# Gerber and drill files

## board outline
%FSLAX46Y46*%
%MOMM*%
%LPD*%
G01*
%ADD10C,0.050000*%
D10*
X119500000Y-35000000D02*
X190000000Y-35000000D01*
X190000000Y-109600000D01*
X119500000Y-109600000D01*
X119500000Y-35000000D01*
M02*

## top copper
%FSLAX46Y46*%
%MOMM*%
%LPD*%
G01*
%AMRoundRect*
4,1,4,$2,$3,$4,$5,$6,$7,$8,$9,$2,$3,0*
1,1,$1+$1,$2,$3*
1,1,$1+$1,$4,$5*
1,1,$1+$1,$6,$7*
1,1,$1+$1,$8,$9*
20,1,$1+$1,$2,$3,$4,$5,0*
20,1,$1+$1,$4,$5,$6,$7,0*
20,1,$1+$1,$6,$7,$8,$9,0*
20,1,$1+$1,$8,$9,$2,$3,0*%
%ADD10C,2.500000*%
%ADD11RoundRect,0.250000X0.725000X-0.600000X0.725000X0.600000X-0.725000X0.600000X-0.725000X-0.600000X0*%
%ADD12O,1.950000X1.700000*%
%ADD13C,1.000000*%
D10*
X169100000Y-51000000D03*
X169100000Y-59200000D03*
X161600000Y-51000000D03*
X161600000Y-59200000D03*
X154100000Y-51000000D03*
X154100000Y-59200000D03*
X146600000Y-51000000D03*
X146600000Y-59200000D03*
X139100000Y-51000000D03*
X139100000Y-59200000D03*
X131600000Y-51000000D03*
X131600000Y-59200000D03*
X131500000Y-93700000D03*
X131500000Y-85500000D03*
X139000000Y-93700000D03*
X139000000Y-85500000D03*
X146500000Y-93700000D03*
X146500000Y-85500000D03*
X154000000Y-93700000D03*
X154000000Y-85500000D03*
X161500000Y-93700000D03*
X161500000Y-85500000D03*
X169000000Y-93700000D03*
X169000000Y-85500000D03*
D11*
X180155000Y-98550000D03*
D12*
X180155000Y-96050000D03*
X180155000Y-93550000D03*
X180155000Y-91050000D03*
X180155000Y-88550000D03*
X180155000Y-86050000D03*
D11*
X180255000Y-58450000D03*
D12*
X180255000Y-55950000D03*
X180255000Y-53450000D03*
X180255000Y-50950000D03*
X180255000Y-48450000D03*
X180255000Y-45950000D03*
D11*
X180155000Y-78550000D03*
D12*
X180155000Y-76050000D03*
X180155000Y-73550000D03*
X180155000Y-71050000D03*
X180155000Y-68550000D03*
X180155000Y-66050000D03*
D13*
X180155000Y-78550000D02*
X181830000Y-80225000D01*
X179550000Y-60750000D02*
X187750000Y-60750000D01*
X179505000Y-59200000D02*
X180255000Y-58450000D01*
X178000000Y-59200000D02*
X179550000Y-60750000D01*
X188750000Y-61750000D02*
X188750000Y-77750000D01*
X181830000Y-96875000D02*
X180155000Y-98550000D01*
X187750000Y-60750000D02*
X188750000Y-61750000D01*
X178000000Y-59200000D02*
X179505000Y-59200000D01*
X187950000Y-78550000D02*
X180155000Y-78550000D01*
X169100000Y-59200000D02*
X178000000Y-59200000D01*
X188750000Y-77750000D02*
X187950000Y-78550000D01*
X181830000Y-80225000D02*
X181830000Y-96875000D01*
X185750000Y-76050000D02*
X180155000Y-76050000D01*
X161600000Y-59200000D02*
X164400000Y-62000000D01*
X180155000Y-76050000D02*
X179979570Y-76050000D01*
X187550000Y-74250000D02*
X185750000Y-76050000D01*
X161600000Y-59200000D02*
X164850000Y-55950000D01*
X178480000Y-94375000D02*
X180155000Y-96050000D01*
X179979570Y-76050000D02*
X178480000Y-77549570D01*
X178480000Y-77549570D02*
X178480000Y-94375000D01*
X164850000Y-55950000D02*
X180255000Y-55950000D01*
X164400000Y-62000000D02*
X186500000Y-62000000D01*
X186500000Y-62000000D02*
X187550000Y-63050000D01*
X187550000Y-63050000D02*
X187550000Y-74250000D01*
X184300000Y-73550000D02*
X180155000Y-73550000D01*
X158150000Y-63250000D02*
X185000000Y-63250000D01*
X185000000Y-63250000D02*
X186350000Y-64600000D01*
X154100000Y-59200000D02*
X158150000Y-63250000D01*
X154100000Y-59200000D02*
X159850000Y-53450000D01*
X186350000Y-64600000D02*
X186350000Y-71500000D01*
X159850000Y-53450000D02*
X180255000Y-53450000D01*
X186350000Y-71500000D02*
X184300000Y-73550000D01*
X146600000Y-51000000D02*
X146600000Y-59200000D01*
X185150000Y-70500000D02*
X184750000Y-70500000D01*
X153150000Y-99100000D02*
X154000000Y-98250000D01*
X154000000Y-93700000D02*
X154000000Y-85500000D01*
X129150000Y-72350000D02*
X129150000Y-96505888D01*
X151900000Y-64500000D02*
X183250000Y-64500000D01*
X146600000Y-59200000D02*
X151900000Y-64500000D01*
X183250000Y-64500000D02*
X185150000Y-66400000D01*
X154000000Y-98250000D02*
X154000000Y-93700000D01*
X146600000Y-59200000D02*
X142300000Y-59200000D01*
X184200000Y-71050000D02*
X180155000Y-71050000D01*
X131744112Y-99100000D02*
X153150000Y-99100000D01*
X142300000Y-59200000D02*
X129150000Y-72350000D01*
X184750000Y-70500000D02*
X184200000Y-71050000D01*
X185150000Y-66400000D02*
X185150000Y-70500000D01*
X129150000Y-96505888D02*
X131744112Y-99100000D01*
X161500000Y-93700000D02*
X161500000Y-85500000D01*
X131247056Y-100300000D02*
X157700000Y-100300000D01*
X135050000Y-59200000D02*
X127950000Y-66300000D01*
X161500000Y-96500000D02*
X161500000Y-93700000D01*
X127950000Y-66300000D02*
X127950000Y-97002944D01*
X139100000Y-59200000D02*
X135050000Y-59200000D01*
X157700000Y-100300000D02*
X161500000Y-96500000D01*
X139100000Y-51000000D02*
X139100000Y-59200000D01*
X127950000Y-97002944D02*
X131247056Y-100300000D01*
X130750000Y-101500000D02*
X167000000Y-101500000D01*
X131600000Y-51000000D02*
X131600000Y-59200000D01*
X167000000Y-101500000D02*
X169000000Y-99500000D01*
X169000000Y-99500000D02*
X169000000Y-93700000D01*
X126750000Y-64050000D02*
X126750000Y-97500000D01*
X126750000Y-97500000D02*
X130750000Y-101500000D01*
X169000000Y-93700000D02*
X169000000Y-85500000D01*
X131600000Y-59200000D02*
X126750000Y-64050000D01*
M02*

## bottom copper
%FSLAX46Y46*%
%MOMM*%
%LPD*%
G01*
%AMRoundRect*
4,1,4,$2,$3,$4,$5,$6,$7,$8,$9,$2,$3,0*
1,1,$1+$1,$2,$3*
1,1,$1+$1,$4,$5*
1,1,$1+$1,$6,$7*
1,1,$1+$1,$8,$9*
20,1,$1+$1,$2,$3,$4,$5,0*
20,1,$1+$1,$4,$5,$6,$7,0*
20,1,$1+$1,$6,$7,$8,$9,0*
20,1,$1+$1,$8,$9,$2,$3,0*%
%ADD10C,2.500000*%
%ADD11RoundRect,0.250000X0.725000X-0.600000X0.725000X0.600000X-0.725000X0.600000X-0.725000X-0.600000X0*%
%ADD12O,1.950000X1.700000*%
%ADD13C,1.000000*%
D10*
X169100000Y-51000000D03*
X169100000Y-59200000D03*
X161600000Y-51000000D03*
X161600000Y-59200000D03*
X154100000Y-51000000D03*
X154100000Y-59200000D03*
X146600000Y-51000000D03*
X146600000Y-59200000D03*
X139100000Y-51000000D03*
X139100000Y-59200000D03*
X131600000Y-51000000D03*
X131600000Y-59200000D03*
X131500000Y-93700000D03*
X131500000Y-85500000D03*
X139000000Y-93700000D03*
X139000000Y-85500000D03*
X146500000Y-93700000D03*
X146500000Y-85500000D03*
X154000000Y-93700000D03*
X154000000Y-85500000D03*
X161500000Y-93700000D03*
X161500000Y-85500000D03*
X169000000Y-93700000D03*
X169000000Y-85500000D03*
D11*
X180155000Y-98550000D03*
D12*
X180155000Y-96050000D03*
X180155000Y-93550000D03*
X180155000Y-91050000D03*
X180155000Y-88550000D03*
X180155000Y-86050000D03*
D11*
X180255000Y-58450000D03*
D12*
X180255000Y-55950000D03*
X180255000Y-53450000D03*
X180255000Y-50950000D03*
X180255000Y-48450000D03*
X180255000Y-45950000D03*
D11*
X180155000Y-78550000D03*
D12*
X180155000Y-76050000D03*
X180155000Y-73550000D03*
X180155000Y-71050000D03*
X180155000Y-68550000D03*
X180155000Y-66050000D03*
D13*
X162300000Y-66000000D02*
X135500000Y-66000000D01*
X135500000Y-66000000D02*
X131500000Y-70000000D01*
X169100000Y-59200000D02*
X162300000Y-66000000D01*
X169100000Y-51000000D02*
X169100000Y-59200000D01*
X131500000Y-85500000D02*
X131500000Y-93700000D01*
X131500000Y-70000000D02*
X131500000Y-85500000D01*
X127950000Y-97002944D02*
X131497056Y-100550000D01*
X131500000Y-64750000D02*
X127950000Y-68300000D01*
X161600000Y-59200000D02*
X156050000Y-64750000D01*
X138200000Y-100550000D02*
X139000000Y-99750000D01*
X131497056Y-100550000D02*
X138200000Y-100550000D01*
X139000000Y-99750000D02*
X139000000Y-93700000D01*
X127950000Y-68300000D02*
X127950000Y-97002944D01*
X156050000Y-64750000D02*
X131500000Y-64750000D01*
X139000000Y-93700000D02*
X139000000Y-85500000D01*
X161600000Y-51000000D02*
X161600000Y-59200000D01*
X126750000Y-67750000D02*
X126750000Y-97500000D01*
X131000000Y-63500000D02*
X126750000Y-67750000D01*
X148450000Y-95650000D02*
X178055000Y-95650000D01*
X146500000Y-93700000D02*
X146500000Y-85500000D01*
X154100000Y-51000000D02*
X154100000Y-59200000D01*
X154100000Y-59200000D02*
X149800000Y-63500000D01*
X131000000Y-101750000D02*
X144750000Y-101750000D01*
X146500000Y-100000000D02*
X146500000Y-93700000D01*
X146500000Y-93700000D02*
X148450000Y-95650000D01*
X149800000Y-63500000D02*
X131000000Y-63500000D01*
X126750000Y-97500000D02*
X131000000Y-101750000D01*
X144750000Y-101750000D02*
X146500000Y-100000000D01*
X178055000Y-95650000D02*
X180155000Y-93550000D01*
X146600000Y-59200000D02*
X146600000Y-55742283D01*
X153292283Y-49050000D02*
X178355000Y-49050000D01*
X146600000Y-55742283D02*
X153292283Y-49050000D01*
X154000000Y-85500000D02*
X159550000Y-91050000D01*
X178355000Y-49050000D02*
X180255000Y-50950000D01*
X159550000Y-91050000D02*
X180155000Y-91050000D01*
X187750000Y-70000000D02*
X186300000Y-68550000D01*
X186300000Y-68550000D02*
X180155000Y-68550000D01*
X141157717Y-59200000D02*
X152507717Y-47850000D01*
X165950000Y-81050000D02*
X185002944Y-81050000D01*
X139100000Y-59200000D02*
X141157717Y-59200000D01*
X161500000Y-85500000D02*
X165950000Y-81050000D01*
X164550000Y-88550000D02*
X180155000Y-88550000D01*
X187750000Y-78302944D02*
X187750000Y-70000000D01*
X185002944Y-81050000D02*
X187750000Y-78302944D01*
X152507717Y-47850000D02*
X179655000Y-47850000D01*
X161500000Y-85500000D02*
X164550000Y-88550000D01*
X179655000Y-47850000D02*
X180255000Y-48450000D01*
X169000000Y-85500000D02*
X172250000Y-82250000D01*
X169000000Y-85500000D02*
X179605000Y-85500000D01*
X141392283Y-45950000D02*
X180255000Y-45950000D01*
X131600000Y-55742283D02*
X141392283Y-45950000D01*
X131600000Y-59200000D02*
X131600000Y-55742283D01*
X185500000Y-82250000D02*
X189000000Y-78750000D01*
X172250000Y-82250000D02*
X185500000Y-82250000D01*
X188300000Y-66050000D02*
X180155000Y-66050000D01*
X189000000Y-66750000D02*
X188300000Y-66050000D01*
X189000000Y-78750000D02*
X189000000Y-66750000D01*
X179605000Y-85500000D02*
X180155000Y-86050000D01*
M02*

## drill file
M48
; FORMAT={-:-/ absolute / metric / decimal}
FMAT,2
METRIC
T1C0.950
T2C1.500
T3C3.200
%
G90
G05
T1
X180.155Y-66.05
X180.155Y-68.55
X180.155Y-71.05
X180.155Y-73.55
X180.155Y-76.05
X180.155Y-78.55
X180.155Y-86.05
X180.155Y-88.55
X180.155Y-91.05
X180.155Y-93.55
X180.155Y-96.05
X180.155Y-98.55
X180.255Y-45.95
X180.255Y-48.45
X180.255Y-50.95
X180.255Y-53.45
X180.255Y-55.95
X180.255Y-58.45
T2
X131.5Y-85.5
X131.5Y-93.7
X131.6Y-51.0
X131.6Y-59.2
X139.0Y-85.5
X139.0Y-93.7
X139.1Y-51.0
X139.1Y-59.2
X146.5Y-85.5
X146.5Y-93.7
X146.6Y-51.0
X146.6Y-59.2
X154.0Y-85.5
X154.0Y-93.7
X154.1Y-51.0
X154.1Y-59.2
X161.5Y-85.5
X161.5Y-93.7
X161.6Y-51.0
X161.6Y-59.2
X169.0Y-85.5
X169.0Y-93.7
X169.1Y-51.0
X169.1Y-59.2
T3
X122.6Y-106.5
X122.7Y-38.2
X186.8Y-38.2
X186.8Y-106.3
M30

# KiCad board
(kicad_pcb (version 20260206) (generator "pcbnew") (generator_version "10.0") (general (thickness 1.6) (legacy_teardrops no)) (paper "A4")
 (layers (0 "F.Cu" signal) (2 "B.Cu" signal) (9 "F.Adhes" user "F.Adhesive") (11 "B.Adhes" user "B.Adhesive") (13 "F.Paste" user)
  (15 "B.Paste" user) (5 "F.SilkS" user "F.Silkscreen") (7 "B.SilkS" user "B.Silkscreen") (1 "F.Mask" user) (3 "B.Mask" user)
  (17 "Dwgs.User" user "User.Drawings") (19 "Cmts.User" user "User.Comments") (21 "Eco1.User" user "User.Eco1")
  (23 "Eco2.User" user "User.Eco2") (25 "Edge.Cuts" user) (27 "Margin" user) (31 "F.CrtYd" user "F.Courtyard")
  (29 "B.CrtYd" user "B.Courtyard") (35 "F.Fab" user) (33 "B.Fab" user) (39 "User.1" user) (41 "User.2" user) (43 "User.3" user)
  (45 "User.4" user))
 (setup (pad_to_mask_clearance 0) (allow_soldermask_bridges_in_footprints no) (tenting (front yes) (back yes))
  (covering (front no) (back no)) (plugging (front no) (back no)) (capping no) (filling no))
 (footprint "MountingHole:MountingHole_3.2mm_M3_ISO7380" (layer "F.Cu") (at 122.6 106.5)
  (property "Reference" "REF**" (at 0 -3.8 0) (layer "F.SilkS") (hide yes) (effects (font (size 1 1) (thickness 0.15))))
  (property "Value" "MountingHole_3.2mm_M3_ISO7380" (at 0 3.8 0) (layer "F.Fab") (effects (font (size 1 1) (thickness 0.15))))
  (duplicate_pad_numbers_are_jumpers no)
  (pad "" np_thru_hole circle (at 0 0) (size 3.2 3.2) (drill 3.2) (layers "*.Cu" "*.Mask")))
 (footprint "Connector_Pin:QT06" (layer "F.Cu") (at 150.36 51.82)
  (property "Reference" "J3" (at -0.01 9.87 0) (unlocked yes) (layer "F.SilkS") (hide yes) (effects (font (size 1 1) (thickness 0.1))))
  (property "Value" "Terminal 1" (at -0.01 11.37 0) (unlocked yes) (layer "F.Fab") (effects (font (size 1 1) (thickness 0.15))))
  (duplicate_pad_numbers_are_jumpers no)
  (pad "1" thru_hole circle (at 18.74 -0.82) (size 2.5 2.5) (drill 1.5) (layers "*.Cu" "*.Mask") (remove_unused_layers no)
   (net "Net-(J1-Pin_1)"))
  (pad "1" thru_hole circle (at 18.74 7.38) (size 2.5 2.5) (drill 1.5) (layers "*.Cu" "*.Mask") (remove_unused_layers no)
   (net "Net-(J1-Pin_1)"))
  (pad "2" thru_hole circle (at 11.24 -0.82) (size 2.5 2.5) (drill 1.5) (layers "*.Cu" "*.Mask") (remove_unused_layers no)
   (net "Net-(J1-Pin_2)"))
  (pad "2" thru_hole circle (at 11.24 7.38) (size 2.5 2.5) (drill 1.5) (layers "*.Cu" "*.Mask") (remove_unused_layers no)
   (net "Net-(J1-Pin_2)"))
  (pad "3" thru_hole circle (at 3.74 -0.82) (size 2.5 2.5) (drill 1.5) (layers "*.Cu" "*.Mask") (remove_unused_layers no)
   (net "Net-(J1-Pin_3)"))
  (pad "3" thru_hole circle (at 3.74 7.38) (size 2.5 2.5) (drill 1.5) (layers "*.Cu" "*.Mask") (remove_unused_layers no)
   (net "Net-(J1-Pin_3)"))
  (pad "4" thru_hole circle (at -3.76 -0.82) (size 2.5 2.5) (drill 1.5) (layers "*.Cu" "*.Mask") (remove_unused_layers no)
   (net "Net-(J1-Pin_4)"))
  (pad "4" thru_hole circle (at -3.76 7.38) (size 2.5 2.5) (drill 1.5) (layers "*.Cu" "*.Mask") (remove_unused_layers no)
   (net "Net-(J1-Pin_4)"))
  (pad "5" thru_hole circle (at -11.26 -0.82) (size 2.5 2.5) (drill 1.5) (layers "*.Cu" "*.Mask") (remove_unused_layers no)
   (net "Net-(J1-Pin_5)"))
  (pad "5" thru_hole circle (at -11.26 7.38) (size 2.5 2.5) (drill 1.5) (layers "*.Cu" "*.Mask") (remove_unused_layers no)
   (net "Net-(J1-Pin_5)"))
  (pad "6" thru_hole circle (at -18.76 -0.82) (size 2.5 2.5) (drill 1.5) (layers "*.Cu" "*.Mask") (remove_unused_layers no)
   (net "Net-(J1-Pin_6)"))
  (pad "6" thru_hole circle (at -18.76 7.38) (size 2.5 2.5) (drill 1.5) (layers "*.Cu" "*.Mask") (remove_unused_layers no)
   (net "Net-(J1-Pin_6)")))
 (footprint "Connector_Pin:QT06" (layer "F.Cu") (at 150.24 92.88 180)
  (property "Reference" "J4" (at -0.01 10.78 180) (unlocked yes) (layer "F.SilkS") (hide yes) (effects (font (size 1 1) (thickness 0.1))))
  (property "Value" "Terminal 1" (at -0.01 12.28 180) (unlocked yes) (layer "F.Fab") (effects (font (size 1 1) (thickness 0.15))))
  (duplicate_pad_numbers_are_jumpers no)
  (pad "1" thru_hole circle (at 18.74 -0.82 180) (size 2.5 2.5) (drill 1.5) (layers "*.Cu" "*.Mask") (remove_unused_layers no)
   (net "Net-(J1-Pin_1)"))
  (pad "1" thru_hole circle (at 18.74 7.38 180) (size 2.5 2.5) (drill 1.5) (layers "*.Cu" "*.Mask") (remove_unused_layers no)
   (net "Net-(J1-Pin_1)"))
  (pad "2" thru_hole circle (at 11.24 -0.82 180) (size 2.5 2.5) (drill 1.5) (layers "*.Cu" "*.Mask") (remove_unused_layers no)
   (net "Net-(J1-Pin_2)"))
  (pad "2" thru_hole circle (at 11.24 7.38 180) (size 2.5 2.5) (drill 1.5) (layers "*.Cu" "*.Mask") (remove_unused_layers no)
   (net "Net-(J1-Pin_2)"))
  (pad "3" thru_hole circle (at 3.74 -0.82 180) (size 2.5 2.5) (drill 1.5) (layers "*.Cu" "*.Mask") (remove_unused_layers no)
   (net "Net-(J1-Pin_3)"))
  (pad "3" thru_hole circle (at 3.74 7.38 180) (size 2.5 2.5) (drill 1.5) (layers "*.Cu" "*.Mask") (remove_unused_layers no)
   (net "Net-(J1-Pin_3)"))
  (pad "4" thru_hole circle (at -3.76 -0.82 180) (size 2.5 2.5) (drill 1.5) (layers "*.Cu" "*.Mask") (remove_unused_layers no)
   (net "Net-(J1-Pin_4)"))
  (pad "4" thru_hole circle (at -3.76 7.38 180) (size 2.5 2.5) (drill 1.5) (layers "*.Cu" "*.Mask") (remove_unused_layers no)
   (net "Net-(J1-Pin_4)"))
  (pad "5" thru_hole circle (at -11.26 -0.82 180) (size 2.5 2.5) (drill 1.5) (layers "*.Cu" "*.Mask") (remove_unused_layers no)
   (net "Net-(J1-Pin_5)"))
  (pad "5" thru_hole circle (at -11.26 7.38 180) (size 2.5 2.5) (drill 1.5) (layers "*.Cu" "*.Mask") (remove_unused_layers no)
   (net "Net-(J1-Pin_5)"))
  (pad "6" thru_hole circle (at -18.76 -0.82 180) (size 2.5 2.5) (drill 1.5) (layers "*.Cu" "*.Mask") (remove_unused_layers no)
   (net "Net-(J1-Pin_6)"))
  (pad "6" thru_hole circle (at -18.76 7.38 180) (size 2.5 2.5) (drill 1.5) (layers "*.Cu" "*.Mask") (remove_unused_layers no)
   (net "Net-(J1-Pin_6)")))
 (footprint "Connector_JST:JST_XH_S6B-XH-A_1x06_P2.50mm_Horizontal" (layer "F.Cu") (at 180.155 98.55 90)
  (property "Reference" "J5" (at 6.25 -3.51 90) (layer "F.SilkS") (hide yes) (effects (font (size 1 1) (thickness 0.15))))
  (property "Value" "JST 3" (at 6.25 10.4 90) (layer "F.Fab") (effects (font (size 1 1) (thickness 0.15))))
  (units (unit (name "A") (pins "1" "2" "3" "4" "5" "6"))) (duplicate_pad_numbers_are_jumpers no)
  (pad "1" thru_hole roundrect (at 0 0 90) (size 1.7 1.95) (drill 0.95) (layers "*.Cu" "*.Mask") (remove_unused_layers no)
   (roundrect_rratio 0.147059) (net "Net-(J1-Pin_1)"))
  (pad "2" thru_hole oval (at 2.5 0 90) (size 1.7 1.95) (drill 0.95) (layers "*.Cu" "*.Mask") (remove_unused_layers no)
   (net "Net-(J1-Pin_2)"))
  (pad "3" thru_hole oval (at 5 0 90) (size 1.7 1.95) (drill 0.95) (layers "*.Cu" "*.Mask") (remove_unused_layers no) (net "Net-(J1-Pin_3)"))
  (pad "4" thru_hole oval (at 7.5 0 90) (size 1.7 1.95) (drill 0.95) (layers "*.Cu" "*.Mask") (remove_unused_layers no)
   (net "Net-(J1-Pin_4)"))
  (pad "5" thru_hole oval (at 10 0 90) (size 1.7 1.95) (drill 0.95) (layers "*.Cu" "*.Mask") (remove_unused_layers no)
   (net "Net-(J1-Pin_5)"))
  (pad "6" thru_hole oval (at 12.5 0 90) (size 1.7 1.95) (drill 0.95) (layers "*.Cu" "*.Mask") (remove_unused_layers no)
   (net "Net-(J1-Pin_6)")))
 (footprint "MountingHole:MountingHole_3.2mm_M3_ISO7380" (layer "F.Cu") (at 122.7 38.2)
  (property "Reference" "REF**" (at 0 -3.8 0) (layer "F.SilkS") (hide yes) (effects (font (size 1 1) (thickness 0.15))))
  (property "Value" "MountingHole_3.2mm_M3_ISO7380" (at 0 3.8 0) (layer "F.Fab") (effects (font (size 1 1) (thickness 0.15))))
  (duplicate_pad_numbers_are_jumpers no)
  (pad "" np_thru_hole circle (at 0 0) (size 3.2 3.2) (drill 3.2) (layers "*.Cu" "*.Mask")))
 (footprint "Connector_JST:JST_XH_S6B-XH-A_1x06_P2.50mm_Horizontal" (layer "F.Cu") (at 180.255 58.45 90)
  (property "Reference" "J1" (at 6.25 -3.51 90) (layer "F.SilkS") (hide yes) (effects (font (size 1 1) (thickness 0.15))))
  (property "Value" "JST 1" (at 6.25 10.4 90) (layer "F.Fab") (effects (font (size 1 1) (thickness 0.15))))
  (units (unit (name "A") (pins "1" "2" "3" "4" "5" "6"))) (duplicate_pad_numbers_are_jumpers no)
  (pad "1" thru_hole roundrect (at 0 0 90) (size 1.7 1.95) (drill 0.95) (layers "*.Cu" "*.Mask") (remove_unused_layers no)
   (roundrect_rratio 0.147059) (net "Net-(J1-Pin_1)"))
  (pad "2" thru_hole oval (at 2.5 0 90) (size 1.7 1.95) (drill 0.95) (layers "*.Cu" "*.Mask") (remove_unused_layers no)
   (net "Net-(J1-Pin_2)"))
  (pad "3" thru_hole oval (at 5 0 90) (size 1.7 1.95) (drill 0.95) (layers "*.Cu" "*.Mask") (remove_unused_layers no) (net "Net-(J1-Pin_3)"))
  (pad "4" thru_hole oval (at 7.5 0 90) (size 1.7 1.95) (drill 0.95) (layers "*.Cu" "*.Mask") (remove_unused_layers no)
   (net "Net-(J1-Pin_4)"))
  (pad "5" thru_hole oval (at 10 0 90) (size 1.7 1.95) (drill 0.95) (layers "*.Cu" "*.Mask") (remove_unused_layers no)
   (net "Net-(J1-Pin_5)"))
  (pad "6" thru_hole oval (at 12.5 0 90) (size 1.7 1.95) (drill 0.95) (layers "*.Cu" "*.Mask") (remove_unused_layers no)
   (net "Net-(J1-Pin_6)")))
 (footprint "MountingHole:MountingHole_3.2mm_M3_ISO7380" (layer "F.Cu") (at 186.8 106.3)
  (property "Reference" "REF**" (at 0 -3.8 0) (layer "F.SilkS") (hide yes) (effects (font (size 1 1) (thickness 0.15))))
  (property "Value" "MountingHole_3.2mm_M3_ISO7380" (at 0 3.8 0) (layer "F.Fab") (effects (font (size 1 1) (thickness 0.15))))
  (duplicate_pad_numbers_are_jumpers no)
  (pad "" np_thru_hole circle (at 0 0) (size 3.2 3.2) (drill 3.2) (layers "*.Cu" "*.Mask")))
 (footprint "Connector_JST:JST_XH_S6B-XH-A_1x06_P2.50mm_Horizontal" (layer "F.Cu") (at 180.155 78.55 90)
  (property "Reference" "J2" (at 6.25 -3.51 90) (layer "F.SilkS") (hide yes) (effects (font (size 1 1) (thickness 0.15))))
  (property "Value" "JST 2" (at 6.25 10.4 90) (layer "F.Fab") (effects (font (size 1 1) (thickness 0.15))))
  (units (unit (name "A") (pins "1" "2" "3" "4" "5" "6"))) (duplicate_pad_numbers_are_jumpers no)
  (pad "1" thru_hole roundrect (at 0 0 90) (size 1.7 1.95) (drill 0.95) (layers "*.Cu" "*.Mask") (remove_unused_layers no)
   (roundrect_rratio 0.147059) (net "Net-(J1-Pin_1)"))
  (pad "2" thru_hole oval (at 2.5 0 90) (size 1.7 1.95) (drill 0.95) (layers "*.Cu" "*.Mask") (remove_unused_layers no)
   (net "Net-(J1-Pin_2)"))
  (pad "3" thru_hole oval (at 5 0 90) (size 1.7 1.95) (drill 0.95) (layers "*.Cu" "*.Mask") (remove_unused_layers no) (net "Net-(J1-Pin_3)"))
  (pad "4" thru_hole oval (at 7.5 0 90) (size 1.7 1.95) (drill 0.95) (layers "*.Cu" "*.Mask") (remove_unused_layers no)
   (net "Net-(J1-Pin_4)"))
  (pad "5" thru_hole oval (at 10 0 90) (size 1.7 1.95) (drill 0.95) (layers "*.Cu" "*.Mask") (remove_unused_layers no)
   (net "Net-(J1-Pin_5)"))
  (pad "6" thru_hole oval (at 12.5 0 90) (size 1.7 1.95) (drill 0.95) (layers "*.Cu" "*.Mask") (remove_unused_layers no)
   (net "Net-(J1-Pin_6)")))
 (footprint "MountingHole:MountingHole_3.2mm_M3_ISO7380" (layer "F.Cu") (at 186.8 38.2)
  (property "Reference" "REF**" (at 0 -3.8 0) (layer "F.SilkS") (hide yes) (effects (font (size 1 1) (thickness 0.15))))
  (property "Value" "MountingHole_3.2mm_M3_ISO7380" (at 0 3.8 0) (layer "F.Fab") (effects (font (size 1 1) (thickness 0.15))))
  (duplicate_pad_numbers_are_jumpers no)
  (pad "" np_thru_hole circle (at 0 0) (size 3.2 3.2) (drill 3.2) (layers "*.Cu" "*.Mask")))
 (gr_rect (start 119.5 35) (end 190 109.6) (stroke (width 0.05) (type default)) (fill no) (layer "Edge.Cuts"))
 (segment (start 180.155 78.55) (end 181.83 80.225) (width 1) (layer "F.Cu") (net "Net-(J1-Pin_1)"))
 (segment (start 179.55 60.75) (end 187.75 60.75) (width 1) (layer "F.Cu") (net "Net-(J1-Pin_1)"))
 (segment (start 179.505 59.2) (end 180.255 58.45) (width 1) (layer "F.Cu") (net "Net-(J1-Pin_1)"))
 (segment (start 178 59.2) (end 179.55 60.75) (width 1) (layer "F.Cu") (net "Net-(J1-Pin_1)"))
 (segment (start 188.75 61.75) (end 188.75 77.75) (width 1) (layer "F.Cu") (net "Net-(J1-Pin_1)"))
 (segment (start 181.83 96.875) (end 180.155 98.55) (width 1) (layer "F.Cu") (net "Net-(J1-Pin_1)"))
 (segment (start 187.75 60.75) (end 188.75 61.75) (width 1) (layer "F.Cu") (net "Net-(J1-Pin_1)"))
 (segment (start 178 59.2) (end 179.505 59.2) (width 1) (layer "F.Cu") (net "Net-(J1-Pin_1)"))
 (segment (start 187.95 78.55) (end 180.155 78.55) (width 1) (layer "F.Cu") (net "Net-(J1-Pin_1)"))
 (segment (start 169.1 59.2) (end 178 59.2) (width 1) (layer "F.Cu") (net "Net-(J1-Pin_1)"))
 (segment (start 188.75 77.75) (end 187.95 78.55) (width 1) (layer "F.Cu") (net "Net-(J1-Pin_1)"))
 (segment (start 181.83 80.225) (end 181.83 96.875) (width 1) (layer "F.Cu") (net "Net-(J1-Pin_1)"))
 (segment (start 162.3 66) (end 135.5 66) (width 1) (layer "B.Cu") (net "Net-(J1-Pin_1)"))
 (segment (start 135.5 66) (end 131.5 70) (width 1) (layer "B.Cu") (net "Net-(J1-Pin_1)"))
 (segment (start 169.1 59.2) (end 162.3 66) (width 1) (layer "B.Cu") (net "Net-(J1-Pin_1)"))
 (segment (start 169.1 51) (end 169.1 59.2) (width 1) (layer "B.Cu") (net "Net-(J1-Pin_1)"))
 (segment (start 131.5 85.5) (end 131.5 93.7) (width 1) (layer "B.Cu") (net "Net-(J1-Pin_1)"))
 (segment (start 131.5 70) (end 131.5 85.5) (width 1) (layer "B.Cu") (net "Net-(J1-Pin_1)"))
 (segment (start 185.75 76.05) (end 180.155 76.05) (width 1) (layer "F.Cu") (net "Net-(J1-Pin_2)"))
 (segment (start 161.6 59.2) (end 164.4 62) (width 1) (layer "F.Cu") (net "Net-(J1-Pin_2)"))
 (segment (start 180.155 76.05) (end 179.97957 76.05) (width 1) (layer "F.Cu") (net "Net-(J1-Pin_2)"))
 (segment (start 187.55 74.25) (end 185.75 76.05) (width 1) (layer "F.Cu") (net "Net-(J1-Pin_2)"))
 (segment (start 161.6 59.2) (end 164.85 55.95) (width 1) (layer "F.Cu") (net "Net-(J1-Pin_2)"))
 (segment (start 178.48 94.375) (end 180.155 96.05) (width 1) (layer "F.Cu") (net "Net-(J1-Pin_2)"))
 (segment (start 179.97957 76.05) (end 178.48 77.54957) (width 1) (layer "F.Cu") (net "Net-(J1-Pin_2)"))
 (segment (start 178.48 77.54957) (end 178.48 94.375) (width 1) (layer "F.Cu") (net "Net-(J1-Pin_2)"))
 (segment (start 164.85 55.95) (end 180.255 55.95) (width 1) (layer "F.Cu") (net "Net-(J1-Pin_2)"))
 (segment (start 164.4 62) (end 186.5 62) (width 1) (layer "F.Cu") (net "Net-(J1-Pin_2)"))
 (segment (start 186.5 62) (end 187.55 63.05) (width 1) (layer "F.Cu") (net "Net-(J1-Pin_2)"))
 (segment (start 187.55 63.05) (end 187.55 74.25) (width 1) (layer "F.Cu") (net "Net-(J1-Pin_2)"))
 (segment (start 127.95 97.002944) (end 131.497056 100.55) (width 1) (layer "B.Cu") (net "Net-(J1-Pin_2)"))
 (segment (start 131.5 64.75) (end 127.95 68.3) (width 1) (layer "B.Cu") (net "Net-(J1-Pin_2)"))
 (segment (start 161.6 59.2) (end 156.05 64.75) (width 1) (layer "B.Cu") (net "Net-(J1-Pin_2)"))
 (segment (start 138.2 100.55) (end 139 99.75) (width 1) (layer "B.Cu") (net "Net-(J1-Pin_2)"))
 (segment (start 131.497056 100.55) (end 138.2 100.55) (width 1) (layer "B.Cu") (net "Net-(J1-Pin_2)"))
 (segment (start 139 99.75) (end 139 93.7) (width 1) (layer "B.Cu") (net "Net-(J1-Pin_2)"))
 (segment (start 127.95 68.3) (end 127.95 97.002944) (width 1) (layer "B.Cu") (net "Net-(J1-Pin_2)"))
 (segment (start 156.05 64.75) (end 131.5 64.75) (width 1) (layer "B.Cu") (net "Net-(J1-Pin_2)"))
 (segment (start 139 93.7) (end 139 85.5) (width 1) (layer "B.Cu") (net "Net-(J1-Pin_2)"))
 (segment (start 161.6 51) (end 161.6 59.2) (width 1) (layer "B.Cu") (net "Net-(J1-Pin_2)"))
 (segment (start 184.3 73.55) (end 180.155 73.55) (width 1) (layer "F.Cu") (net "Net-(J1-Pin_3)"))
 (segment (start 158.15 63.25) (end 185 63.25) (width 1) (layer "F.Cu") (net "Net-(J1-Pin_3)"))
 (segment (start 185 63.25) (end 186.35 64.6) (width 1) (layer "F.Cu") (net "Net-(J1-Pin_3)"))
 (segment (start 154.1 59.2) (end 158.15 63.25) (width 1) (layer "F.Cu") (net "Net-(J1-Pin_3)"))
 (segment (start 154.1 59.2) (end 159.85 53.45) (width 1) (layer "F.Cu") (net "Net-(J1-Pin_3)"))
 (segment (start 186.35 64.6) (end 186.35 71.5) (width 1) (layer "F.Cu") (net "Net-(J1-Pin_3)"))
 (segment (start 159.85 53.45) (end 180.255 53.45) (width 1) (layer "F.Cu") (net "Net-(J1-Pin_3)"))
 (segment (start 186.35 71.5) (end 184.3 73.55) (width 1) (layer "F.Cu") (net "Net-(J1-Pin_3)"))
 (segment (start 126.75 67.75) (end 126.75 97.5) (width 1) (layer "B.Cu") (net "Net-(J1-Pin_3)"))
 (segment (start 131 63.5) (end 126.75 67.75) (width 1) (layer "B.Cu") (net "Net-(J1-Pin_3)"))
 (segment (start 148.45 95.65) (end 178.055 95.65) (width 1) (layer "B.Cu") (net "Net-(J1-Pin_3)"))
 (segment (start 146.5 93.7) (end 146.5 85.5) (width 1) (layer "B.Cu") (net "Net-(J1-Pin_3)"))
 (segment (start 154.1 51) (end 154.1 59.2) (width 1) (layer "B.Cu") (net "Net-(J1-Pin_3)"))
 (segment (start 154.1 59.2) (end 149.8 63.5) (width 1) (layer "B.Cu") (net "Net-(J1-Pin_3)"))
 (segment (start 131 101.75) (end 144.75 101.75) (width 1) (layer "B.Cu") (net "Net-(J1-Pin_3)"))
 (segment (start 146.5 100) (end 146.5 93.7) (width 1) (layer "B.Cu") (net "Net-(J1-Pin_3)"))
 (segment (start 146.5 93.7) (end 148.45 95.65) (width 1) (layer "B.Cu") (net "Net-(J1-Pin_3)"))
 (segment (start 149.8 63.5) (end 131 63.5) (width 1) (layer "B.Cu") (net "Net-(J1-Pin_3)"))
 (segment (start 126.75 97.5) (end 131 101.75) (width 1) (layer "B.Cu") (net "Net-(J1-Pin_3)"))
 (segment (start 144.75 101.75) (end 146.5 100) (width 1) (layer "B.Cu") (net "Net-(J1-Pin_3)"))
 (segment (start 178.055 95.65) (end 180.155 93.55) (width 1) (layer "B.Cu") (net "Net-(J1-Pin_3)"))
 (segment (start 146.6 51) (end 146.6 59.2) (width 1) (layer "F.Cu") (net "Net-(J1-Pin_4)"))
 (segment (start 185.15 70.5) (end 184.75 70.5) (width 1) (layer "F.Cu") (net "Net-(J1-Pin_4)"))
 (segment (start 153.15 99.1) (end 154 98.25) (width 1) (layer "F.Cu") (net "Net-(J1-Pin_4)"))
 (segment (start 154 93.7) (end 154 85.5) (width 1) (layer "F.Cu") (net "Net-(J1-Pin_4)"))
 (segment (start 129.15 72.35) (end 129.15 96.505888) (width 1) (layer "F.Cu") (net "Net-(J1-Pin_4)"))
 (segment (start 151.9 64.5) (end 183.25 64.5) (width 1) (layer "F.Cu") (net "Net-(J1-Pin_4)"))
 (segment (start 146.6 59.2) (end 151.9 64.5) (width 1) (layer "F.Cu") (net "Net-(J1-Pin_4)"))
 (segment (start 183.25 64.5) (end 185.15 66.4) (width 1) (layer "F.Cu") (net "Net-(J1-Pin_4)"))
 (segment (start 154 98.25) (end 154 93.7) (width 1) (layer "F.Cu") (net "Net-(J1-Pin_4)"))
 (segment (start 146.6 59.2) (end 142.3 59.2) (width 1) (layer "F.Cu") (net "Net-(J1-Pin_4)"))
 (segment (start 184.2 71.05) (end 180.155 71.05) (width 1) (layer "F.Cu") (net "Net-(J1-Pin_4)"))
 (segment (start 131.744112 99.1) (end 153.15 99.1) (width 1) (layer "F.Cu") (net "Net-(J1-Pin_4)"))
 (segment (start 142.3 59.2) (end 129.15 72.35) (width 1) (layer "F.Cu") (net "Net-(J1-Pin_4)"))
 (segment (start 184.75 70.5) (end 184.2 71.05) (width 1) (layer "F.Cu") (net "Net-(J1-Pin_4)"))
 (segment (start 185.15 66.4) (end 185.15 70.5) (width 1) (layer "F.Cu") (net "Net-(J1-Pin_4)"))
 (segment (start 129.15 96.505888) (end 131.744112 99.1) (width 1) (layer "F.Cu") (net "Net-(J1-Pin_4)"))
 (segment (start 146.6 59.2) (end 146.6 55.742283) (width 1) (layer "B.Cu") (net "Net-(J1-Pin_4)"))
 (segment (start 153.292283 49.05) (end 178.355 49.05) (width 1) (layer "B.Cu") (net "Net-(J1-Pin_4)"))
 (segment (start 146.6 55.742283) (end 153.292283 49.05) (width 1) (layer "B.Cu") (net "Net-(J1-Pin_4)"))
 (segment (start 154 85.5) (end 159.55 91.05) (width 1) (layer "B.Cu") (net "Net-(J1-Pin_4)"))
 (segment (start 178.355 49.05) (end 180.255 50.95) (width 1) (layer "B.Cu") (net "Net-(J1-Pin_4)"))
 (segment (start 159.55 91.05) (end 180.155 91.05) (width 1) (layer "B.Cu") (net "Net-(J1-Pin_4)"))
 (segment (start 161.5 93.7) (end 161.5 85.5) (width 1) (layer "F.Cu") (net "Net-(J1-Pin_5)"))
 (segment (start 131.247056 100.3) (end 157.7 100.3) (width 1) (layer "F.Cu") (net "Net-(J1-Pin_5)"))
 (segment (start 135.05 59.2) (end 127.95 66.3) (width 1) (layer "F.Cu") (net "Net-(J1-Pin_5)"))
 (segment (start 161.5 96.5) (end 161.5 93.7) (width 1) (layer "F.Cu") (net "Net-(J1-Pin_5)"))
 (segment (start 127.95 66.3) (end 127.95 97.002944) (width 1) (layer "F.Cu") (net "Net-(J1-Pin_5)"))
 (segment (start 139.1 59.2) (end 135.05 59.2) (width 1) (layer "F.Cu") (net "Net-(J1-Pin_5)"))
 (segment (start 157.7 100.3) (end 161.5 96.5) (width 1) (layer "F.Cu") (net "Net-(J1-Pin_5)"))
 (segment (start 139.1 51) (end 139.1 59.2) (width 1) (layer "F.Cu") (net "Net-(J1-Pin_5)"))
 (segment (start 127.95 97.002944) (end 131.247056 100.3) (width 1) (layer "F.Cu") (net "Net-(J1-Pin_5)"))
 (segment (start 187.75 70) (end 186.3 68.55) (width 1) (layer "B.Cu") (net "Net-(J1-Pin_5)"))
 (segment (start 186.3 68.55) (end 180.155 68.55) (width 1) (layer "B.Cu") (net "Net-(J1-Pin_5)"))
 (segment (start 141.157717 59.2) (end 152.507717 47.85) (width 1) (layer "B.Cu") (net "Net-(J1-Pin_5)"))
 (segment (start 165.95 81.05) (end 185.002944 81.05) (width 1) (layer "B.Cu") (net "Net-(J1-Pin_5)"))
 (segment (start 139.1 59.2) (end 141.157717 59.2) (width 1) (layer "B.Cu") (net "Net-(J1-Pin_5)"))
 (segment (start 161.5 85.5) (end 165.95 81.05) (width 1) (layer "B.Cu") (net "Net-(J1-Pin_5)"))
 (segment (start 164.55 88.55) (end 180.155 88.55) (width 1) (layer "B.Cu") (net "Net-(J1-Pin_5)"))
 (segment (start 187.75 78.302944) (end 187.75 70) (width 1) (layer "B.Cu") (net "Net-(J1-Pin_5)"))
 (segment (start 185.002944 81.05) (end 187.75 78.302944) (width 1) (layer "B.Cu") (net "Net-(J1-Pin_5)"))
 (segment (start 152.507717 47.85) (end 179.655 47.85) (width 1) (layer "B.Cu") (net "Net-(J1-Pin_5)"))
 (segment (start 161.5 85.5) (end 164.55 88.55) (width 1) (layer "B.Cu") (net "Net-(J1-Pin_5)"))
 (segment (start 179.655 47.85) (end 180.255 48.45) (width 1) (layer "B.Cu") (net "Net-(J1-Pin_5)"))
 (segment (start 130.75 101.5) (end 167 101.5) (width 1) (layer "F.Cu") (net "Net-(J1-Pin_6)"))
 (segment (start 131.6 51) (end 131.6 59.2) (width 1) (layer "F.Cu") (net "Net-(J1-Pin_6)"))
 (segment (start 167 101.5) (end 169 99.5) (width 1) (layer "F.Cu") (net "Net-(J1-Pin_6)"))
 (segment (start 169 99.5) (end 169 93.7) (width 1) (layer "F.Cu") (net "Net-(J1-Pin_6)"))
 (segment (start 126.75 64.05) (end 126.75 97.5) (width 1) (layer "F.Cu") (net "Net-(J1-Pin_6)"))
 (segment (start 126.75 97.5) (end 130.75 101.5) (width 1) (layer "F.Cu") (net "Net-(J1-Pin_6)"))
 (segment (start 169 93.7) (end 169 85.5) (width 1) (layer "F.Cu") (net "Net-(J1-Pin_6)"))
 (segment (start 131.6 59.2) (end 126.75 64.05) (width 1) (layer "F.Cu") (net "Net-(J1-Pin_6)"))
 (segment (start 169 85.5) (end 172.25 82.25) (width 1) (layer "B.Cu") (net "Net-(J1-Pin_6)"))
 (segment (start 169 85.5) (end 179.605 85.5) (width 1) (layer "B.Cu") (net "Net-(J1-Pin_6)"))
 (segment (start 141.392283 45.95) (end 180.255 45.95) (width 1) (layer "B.Cu") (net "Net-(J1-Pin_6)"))
 (segment (start 131.6 55.742283) (end 141.392283 45.95) (width 1) (layer "B.Cu") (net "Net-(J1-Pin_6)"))
 (segment (start 131.6 59.2) (end 131.6 55.742283) (width 1) (layer "B.Cu") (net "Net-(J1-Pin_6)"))
 (segment (start 185.5 82.25) (end 189 78.75) (width 1) (layer "B.Cu") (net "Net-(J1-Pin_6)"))
 (segment (start 172.25 82.25) (end 185.5 82.25) (width 1) (layer "B.Cu") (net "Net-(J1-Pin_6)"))
 (segment (start 188.3 66.05) (end 180.155 66.05) (width 1) (layer "B.Cu") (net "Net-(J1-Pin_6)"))
 (segment (start 189 66.75) (end 188.3 66.05) (width 1) (layer "B.Cu") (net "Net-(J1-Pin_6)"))
 (segment (start 189 78.75) (end 189 66.75) (width 1) (layer "B.Cu") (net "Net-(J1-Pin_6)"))
 (segment (start 179.605 85.5) (end 180.155 86.05) (width 1) (layer "B.Cu") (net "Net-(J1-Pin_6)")))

